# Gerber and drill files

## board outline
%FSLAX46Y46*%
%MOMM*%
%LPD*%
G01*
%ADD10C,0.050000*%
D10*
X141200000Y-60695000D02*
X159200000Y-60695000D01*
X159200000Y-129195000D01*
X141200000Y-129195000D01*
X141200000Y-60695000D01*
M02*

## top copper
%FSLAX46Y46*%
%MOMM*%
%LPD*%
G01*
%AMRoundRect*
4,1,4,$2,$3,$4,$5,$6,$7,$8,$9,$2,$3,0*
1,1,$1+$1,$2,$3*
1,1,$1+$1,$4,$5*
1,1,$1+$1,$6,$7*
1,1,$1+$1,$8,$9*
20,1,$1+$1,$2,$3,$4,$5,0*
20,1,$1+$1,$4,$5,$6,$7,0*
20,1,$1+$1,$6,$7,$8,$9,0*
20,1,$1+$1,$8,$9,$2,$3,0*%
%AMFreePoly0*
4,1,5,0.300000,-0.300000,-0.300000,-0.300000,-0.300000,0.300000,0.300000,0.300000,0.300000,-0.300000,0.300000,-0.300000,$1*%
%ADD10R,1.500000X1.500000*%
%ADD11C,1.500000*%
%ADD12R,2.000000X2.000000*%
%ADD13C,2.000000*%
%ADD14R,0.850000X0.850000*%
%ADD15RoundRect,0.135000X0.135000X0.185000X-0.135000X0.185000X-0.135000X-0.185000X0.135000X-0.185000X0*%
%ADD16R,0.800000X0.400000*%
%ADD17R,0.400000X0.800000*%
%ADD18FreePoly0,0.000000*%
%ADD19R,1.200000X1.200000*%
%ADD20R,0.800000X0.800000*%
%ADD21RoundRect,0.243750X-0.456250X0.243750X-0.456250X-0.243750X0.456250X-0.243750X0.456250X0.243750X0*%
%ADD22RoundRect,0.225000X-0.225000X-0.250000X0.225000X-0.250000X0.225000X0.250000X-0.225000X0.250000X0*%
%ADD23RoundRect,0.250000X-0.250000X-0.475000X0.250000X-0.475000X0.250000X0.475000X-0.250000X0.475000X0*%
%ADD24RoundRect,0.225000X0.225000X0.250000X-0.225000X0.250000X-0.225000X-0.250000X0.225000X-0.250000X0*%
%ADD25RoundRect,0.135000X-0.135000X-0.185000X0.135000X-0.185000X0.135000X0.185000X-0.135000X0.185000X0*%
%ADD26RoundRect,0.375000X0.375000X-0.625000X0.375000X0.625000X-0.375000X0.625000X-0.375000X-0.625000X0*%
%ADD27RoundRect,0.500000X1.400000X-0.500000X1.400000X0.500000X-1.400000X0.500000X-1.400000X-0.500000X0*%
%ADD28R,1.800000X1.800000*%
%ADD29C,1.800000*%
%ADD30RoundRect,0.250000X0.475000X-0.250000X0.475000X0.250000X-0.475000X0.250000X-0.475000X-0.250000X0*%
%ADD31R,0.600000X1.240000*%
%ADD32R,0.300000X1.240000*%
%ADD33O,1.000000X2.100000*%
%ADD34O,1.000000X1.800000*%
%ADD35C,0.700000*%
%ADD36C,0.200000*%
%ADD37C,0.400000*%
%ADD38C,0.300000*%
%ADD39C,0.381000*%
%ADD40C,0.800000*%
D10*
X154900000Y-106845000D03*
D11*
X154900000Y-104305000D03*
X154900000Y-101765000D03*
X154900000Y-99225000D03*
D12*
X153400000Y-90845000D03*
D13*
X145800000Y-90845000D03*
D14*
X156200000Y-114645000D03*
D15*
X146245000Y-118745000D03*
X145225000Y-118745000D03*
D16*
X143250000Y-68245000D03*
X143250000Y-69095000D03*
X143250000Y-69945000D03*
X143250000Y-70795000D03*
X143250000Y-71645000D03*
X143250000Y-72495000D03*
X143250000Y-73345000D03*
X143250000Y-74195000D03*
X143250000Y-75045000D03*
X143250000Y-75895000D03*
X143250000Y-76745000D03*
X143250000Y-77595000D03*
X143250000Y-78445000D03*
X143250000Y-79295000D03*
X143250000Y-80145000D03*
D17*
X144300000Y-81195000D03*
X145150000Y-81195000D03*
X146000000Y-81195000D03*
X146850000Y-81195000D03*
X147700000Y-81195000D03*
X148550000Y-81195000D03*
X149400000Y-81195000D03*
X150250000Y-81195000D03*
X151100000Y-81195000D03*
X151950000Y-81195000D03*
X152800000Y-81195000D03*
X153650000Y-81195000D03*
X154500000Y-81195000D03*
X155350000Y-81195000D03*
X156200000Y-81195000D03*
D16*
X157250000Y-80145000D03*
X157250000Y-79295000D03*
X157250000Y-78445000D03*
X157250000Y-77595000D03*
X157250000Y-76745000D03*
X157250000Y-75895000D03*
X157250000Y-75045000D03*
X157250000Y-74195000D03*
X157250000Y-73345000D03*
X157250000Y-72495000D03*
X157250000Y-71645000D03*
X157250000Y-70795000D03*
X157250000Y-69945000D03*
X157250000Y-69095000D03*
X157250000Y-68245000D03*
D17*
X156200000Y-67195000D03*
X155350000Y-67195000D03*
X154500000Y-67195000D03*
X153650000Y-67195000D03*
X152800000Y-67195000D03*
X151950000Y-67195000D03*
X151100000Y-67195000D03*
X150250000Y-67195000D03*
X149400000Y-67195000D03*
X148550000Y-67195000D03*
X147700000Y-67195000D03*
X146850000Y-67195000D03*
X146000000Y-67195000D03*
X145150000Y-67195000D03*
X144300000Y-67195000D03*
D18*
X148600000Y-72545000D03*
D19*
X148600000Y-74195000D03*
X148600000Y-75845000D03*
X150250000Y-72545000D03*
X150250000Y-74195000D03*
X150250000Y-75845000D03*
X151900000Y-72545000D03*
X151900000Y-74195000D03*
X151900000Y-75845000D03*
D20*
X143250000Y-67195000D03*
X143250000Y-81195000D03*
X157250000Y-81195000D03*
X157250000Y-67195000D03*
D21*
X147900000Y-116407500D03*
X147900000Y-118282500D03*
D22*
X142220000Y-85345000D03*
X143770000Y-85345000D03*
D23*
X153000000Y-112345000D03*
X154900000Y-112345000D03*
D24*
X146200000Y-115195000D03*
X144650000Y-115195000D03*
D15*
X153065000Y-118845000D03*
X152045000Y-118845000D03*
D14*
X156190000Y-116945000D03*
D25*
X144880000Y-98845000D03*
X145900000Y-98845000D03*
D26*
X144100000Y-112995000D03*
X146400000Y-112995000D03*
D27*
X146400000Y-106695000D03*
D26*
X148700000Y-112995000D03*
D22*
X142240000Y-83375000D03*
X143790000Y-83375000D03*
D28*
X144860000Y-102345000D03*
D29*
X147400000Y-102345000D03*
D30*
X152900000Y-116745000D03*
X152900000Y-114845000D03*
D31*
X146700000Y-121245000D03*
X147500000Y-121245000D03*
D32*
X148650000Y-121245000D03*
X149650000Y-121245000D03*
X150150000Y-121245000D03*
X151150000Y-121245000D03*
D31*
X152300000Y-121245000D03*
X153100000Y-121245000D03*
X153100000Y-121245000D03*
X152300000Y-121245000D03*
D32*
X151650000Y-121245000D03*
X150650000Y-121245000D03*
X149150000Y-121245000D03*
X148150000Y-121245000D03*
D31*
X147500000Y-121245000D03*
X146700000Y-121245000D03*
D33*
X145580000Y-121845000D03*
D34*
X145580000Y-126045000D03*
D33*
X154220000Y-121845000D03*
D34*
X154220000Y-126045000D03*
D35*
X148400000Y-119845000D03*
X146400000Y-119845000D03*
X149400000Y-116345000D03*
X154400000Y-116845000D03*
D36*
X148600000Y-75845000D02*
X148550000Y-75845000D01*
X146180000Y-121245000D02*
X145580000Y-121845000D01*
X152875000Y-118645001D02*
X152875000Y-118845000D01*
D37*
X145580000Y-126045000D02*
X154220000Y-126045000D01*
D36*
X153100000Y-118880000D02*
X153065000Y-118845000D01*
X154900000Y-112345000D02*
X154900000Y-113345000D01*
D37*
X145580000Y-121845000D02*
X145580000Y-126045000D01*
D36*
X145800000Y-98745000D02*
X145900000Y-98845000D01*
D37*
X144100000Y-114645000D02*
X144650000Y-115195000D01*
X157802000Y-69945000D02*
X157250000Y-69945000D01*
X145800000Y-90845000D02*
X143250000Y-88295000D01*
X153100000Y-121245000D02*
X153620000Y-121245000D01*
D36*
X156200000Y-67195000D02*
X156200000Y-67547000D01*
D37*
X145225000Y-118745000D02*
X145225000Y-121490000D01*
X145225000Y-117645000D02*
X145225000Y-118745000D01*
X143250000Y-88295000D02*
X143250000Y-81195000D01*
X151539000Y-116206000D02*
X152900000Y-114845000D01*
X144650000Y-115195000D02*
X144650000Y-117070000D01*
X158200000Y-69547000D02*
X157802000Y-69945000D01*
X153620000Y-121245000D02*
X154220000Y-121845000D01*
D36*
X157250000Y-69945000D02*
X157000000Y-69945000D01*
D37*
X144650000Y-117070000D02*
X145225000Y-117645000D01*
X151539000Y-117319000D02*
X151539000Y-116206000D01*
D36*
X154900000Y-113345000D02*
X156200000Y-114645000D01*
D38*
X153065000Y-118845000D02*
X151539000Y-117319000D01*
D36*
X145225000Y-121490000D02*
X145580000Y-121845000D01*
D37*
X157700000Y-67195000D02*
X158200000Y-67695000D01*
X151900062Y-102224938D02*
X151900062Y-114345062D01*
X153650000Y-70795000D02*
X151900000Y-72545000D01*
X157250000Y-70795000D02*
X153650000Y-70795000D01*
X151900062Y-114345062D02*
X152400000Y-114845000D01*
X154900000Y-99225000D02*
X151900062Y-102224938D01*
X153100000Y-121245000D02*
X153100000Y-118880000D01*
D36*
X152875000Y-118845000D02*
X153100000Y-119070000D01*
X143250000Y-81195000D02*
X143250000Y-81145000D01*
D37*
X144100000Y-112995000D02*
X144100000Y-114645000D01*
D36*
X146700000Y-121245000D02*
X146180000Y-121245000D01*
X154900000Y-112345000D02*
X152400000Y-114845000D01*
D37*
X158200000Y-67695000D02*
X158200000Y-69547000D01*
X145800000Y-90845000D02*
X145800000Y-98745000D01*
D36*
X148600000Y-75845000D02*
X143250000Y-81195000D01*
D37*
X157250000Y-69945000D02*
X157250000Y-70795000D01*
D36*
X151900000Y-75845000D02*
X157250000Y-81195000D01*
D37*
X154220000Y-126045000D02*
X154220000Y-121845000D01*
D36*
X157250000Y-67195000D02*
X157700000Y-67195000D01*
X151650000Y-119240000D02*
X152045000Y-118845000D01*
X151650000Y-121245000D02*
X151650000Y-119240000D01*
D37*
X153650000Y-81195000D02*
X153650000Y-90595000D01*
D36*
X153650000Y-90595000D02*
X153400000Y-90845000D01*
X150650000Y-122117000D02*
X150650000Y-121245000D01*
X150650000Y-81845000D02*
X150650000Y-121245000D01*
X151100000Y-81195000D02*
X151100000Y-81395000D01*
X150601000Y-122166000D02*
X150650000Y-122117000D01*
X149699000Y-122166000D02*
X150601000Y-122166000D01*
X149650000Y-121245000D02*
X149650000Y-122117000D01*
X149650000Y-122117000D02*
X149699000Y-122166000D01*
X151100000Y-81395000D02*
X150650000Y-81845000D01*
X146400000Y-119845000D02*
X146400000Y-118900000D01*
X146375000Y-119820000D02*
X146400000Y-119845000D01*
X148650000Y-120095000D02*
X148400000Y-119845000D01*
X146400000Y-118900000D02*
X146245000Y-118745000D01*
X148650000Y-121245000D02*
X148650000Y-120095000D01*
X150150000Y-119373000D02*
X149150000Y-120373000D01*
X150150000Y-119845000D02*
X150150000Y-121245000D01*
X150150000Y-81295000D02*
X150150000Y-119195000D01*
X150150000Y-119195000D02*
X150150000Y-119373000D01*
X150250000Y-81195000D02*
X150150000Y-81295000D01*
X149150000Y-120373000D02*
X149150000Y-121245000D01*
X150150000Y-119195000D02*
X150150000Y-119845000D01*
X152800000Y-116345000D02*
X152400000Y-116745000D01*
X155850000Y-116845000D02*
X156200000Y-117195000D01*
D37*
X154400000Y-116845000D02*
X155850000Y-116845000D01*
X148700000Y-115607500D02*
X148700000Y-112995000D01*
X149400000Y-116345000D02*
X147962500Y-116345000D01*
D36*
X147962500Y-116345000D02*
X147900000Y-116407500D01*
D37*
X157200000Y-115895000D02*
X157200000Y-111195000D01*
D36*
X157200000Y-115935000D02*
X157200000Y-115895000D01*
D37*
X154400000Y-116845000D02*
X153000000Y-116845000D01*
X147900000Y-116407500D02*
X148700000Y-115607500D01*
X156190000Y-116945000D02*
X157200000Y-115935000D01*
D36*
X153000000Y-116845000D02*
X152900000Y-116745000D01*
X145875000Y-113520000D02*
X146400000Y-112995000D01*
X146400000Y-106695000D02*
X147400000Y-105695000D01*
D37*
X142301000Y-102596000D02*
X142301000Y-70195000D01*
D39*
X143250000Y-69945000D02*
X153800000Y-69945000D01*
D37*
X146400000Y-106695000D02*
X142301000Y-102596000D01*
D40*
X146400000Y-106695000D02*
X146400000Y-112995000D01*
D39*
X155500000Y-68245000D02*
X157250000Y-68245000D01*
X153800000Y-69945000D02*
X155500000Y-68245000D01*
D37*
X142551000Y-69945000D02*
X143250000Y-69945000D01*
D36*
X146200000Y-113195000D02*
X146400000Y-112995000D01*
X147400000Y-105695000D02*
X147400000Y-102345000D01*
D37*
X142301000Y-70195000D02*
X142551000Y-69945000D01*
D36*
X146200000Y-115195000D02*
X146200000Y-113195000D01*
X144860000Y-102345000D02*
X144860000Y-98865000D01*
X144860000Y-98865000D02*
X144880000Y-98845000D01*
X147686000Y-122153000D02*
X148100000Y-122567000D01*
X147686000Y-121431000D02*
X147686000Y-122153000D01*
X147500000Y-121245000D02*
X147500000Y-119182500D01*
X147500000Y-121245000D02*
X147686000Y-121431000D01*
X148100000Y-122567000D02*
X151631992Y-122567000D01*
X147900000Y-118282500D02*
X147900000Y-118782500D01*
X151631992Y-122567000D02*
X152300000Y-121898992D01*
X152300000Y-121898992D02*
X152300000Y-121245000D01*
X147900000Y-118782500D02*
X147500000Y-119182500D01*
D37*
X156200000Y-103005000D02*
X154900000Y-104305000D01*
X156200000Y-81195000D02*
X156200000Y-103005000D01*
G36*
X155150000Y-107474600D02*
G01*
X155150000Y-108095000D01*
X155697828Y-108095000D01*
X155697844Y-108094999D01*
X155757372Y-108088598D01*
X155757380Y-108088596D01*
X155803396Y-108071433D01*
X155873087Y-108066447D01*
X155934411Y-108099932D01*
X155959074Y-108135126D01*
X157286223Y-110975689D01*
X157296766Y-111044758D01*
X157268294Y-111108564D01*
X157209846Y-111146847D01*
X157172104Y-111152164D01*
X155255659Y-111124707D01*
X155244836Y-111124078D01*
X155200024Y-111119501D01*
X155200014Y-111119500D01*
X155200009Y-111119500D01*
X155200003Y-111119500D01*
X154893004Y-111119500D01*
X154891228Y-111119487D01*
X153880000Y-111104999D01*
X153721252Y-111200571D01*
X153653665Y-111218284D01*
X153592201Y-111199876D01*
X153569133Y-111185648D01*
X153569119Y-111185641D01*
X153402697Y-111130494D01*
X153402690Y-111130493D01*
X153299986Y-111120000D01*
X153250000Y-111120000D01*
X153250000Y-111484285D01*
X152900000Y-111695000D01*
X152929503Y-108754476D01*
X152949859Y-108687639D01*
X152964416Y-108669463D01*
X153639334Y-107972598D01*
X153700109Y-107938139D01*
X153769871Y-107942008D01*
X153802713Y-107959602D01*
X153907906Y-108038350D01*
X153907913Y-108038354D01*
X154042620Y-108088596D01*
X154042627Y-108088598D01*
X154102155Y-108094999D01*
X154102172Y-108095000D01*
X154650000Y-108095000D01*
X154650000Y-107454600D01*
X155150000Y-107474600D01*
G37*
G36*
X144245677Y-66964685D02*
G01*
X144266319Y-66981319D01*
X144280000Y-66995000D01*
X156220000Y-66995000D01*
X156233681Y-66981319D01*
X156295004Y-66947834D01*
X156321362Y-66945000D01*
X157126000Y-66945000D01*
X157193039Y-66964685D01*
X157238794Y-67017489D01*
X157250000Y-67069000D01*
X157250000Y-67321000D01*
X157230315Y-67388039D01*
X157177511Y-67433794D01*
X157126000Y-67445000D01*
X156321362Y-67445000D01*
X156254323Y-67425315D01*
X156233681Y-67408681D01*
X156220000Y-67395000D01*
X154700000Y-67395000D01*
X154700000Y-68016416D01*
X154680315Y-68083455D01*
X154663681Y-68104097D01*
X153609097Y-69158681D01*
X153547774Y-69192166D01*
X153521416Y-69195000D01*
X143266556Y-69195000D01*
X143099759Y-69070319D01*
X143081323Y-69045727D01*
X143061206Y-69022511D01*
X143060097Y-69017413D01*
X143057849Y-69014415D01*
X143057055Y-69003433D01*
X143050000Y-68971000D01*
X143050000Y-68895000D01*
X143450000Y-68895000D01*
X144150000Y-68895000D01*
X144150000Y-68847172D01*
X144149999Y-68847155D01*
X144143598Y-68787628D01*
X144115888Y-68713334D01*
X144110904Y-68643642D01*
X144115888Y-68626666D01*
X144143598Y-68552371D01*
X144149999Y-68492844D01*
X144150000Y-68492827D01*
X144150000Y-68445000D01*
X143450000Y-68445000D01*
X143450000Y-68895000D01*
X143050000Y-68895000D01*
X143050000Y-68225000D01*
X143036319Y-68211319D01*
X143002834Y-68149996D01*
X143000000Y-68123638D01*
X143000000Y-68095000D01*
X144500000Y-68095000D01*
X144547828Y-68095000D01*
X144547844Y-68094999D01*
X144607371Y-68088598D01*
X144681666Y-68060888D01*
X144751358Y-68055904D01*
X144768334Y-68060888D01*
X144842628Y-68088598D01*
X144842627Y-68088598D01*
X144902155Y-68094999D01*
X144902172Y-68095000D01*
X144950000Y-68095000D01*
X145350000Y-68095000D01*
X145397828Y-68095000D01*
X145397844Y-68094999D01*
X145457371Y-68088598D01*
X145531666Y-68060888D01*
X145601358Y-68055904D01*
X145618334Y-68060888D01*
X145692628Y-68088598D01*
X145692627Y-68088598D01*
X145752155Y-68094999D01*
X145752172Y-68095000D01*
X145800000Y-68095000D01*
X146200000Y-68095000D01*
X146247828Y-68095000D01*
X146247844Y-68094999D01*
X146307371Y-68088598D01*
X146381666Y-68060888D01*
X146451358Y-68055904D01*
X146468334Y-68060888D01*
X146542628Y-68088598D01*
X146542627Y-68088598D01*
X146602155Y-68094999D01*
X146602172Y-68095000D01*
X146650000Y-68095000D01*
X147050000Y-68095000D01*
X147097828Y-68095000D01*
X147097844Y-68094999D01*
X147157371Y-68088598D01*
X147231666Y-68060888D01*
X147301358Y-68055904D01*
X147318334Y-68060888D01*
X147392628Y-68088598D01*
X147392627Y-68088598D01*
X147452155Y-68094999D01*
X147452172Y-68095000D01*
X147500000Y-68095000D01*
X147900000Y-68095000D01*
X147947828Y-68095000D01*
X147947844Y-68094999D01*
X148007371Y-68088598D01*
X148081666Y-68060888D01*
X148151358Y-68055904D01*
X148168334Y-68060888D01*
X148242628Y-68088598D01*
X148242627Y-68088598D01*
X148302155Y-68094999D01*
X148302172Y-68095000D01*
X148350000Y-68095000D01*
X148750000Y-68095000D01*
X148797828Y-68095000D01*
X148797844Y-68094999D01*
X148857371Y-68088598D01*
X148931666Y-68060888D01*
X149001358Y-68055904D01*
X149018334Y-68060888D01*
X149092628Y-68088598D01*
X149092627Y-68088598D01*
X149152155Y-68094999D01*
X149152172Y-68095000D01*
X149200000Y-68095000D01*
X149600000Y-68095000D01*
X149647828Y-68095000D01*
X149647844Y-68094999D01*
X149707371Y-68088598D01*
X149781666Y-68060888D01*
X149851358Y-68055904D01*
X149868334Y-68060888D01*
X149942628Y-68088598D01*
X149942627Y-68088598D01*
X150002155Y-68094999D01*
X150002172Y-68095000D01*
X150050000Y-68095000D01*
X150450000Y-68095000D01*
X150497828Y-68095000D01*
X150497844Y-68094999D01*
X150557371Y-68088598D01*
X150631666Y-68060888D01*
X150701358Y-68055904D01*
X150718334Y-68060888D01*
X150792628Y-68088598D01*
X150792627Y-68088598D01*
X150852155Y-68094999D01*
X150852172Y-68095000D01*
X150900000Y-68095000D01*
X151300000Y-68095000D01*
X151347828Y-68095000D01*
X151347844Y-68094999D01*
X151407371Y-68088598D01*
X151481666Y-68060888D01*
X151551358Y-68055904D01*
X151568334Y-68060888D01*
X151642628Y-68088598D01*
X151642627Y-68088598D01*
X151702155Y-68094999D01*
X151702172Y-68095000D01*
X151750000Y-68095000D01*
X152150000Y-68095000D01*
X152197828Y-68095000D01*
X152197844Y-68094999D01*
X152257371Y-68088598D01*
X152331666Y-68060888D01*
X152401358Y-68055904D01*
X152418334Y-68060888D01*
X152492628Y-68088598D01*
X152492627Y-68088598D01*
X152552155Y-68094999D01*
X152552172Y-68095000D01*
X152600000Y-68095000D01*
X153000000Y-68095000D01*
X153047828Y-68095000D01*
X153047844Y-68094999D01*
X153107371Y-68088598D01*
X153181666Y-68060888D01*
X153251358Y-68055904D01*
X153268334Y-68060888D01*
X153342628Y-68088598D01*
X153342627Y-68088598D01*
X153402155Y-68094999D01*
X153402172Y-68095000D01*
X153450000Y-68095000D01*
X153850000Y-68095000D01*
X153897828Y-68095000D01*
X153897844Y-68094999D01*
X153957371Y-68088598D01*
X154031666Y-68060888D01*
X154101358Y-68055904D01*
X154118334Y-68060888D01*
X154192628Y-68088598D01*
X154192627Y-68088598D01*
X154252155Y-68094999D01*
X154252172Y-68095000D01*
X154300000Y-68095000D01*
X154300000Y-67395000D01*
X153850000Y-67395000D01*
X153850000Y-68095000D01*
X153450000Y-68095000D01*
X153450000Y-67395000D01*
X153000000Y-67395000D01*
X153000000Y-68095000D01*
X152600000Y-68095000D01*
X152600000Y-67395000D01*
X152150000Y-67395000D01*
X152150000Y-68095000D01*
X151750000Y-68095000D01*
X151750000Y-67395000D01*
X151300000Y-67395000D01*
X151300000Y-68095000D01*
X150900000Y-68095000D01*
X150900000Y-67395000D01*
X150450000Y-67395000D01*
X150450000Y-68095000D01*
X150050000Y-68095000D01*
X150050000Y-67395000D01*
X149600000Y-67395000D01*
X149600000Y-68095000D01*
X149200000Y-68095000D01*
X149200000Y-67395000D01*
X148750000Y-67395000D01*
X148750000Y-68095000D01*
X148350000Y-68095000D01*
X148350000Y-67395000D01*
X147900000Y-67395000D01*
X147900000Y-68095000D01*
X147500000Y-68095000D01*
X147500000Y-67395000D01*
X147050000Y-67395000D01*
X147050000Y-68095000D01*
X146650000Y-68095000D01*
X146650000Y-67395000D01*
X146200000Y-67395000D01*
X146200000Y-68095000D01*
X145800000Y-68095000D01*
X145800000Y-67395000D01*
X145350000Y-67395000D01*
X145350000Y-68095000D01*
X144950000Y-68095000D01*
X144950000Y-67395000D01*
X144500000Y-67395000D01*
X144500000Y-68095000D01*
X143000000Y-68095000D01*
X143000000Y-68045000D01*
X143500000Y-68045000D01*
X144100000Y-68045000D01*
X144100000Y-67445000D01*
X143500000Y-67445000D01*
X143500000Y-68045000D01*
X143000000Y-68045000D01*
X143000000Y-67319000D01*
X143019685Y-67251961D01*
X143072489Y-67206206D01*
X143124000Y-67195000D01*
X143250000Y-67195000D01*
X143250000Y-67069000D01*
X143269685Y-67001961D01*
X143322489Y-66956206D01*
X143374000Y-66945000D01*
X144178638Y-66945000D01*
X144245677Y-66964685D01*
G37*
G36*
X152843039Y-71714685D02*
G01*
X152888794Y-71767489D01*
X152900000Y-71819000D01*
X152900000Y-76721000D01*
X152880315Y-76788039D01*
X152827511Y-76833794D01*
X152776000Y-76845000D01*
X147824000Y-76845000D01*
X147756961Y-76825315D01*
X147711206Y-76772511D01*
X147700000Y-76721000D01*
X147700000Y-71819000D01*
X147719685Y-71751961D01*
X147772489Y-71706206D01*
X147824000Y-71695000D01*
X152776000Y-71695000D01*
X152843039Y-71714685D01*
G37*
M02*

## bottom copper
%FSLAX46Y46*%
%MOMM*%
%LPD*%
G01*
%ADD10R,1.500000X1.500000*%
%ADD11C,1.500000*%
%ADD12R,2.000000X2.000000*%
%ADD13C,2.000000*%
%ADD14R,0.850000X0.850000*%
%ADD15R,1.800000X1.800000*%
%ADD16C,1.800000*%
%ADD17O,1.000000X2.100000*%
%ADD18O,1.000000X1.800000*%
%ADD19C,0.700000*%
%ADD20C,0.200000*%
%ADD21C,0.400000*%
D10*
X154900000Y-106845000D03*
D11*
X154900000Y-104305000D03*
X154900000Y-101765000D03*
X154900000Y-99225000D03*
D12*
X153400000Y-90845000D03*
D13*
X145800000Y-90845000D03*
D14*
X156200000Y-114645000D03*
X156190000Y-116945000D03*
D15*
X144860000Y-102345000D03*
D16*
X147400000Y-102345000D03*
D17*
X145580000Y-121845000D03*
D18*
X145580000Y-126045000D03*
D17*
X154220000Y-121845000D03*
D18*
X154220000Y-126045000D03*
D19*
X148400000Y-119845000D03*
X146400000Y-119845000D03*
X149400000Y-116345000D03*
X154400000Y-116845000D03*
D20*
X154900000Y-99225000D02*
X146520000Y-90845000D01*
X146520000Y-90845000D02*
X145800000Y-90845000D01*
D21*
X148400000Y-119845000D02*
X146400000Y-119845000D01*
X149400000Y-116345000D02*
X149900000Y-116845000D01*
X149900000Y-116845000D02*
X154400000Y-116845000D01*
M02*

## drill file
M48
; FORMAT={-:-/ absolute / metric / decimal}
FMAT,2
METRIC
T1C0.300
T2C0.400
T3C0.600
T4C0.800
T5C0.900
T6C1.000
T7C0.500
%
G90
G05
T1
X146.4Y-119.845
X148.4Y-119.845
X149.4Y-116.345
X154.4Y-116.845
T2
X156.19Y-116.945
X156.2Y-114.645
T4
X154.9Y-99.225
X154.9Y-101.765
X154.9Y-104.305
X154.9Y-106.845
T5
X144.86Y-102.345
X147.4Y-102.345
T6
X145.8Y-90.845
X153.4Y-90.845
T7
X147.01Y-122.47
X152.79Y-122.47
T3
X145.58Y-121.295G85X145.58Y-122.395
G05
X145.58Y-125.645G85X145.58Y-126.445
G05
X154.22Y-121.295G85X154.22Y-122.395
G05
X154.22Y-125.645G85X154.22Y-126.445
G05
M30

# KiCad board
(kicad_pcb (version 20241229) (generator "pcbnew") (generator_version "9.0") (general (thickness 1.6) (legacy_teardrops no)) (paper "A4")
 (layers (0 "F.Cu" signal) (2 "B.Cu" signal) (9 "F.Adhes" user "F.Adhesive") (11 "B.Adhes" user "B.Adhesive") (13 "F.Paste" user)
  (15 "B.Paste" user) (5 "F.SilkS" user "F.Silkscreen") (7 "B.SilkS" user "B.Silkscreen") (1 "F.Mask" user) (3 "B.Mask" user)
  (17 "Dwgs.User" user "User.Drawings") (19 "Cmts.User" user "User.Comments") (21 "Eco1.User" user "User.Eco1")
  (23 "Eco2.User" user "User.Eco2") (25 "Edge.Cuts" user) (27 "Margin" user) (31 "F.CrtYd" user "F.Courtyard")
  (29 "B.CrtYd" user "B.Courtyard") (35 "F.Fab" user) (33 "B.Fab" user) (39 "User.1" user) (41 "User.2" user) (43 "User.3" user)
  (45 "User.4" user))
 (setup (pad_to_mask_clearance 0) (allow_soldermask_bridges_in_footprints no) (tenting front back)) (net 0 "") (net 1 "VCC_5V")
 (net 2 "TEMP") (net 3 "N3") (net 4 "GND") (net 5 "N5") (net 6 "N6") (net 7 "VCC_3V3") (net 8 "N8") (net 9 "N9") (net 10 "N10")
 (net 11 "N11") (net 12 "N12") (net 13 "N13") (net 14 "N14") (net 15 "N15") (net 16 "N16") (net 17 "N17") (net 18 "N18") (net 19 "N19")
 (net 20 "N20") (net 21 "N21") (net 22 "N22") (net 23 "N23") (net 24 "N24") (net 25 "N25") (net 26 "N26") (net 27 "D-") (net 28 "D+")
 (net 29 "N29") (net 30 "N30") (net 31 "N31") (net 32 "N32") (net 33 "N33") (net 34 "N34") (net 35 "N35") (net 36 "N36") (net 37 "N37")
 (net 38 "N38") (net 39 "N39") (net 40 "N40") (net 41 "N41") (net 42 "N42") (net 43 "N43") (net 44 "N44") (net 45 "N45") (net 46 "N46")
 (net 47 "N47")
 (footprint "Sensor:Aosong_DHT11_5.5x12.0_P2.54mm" (layer "F.Cu") (at 154.9 106.845 180)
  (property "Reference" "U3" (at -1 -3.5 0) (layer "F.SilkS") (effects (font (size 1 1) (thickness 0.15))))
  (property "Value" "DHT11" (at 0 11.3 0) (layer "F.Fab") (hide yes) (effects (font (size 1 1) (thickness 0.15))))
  (pad "1" thru_hole rect (at 0 0 180) (size 1.5 1.5) (drill 0.8) (layers "*.Cu" "*.Mask") (remove_unused_layers no) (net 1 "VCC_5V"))
  (pad "2" thru_hole circle (at 0 2.54 180) (size 1.5 1.5) (drill 0.8) (layers "*.Cu" "*.Mask") (remove_unused_layers no) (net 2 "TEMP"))
  (pad "3" thru_hole circle (at 0 5.08 180) (size 1.5 1.5) (drill 0.8) (layers "*.Cu" "*.Mask") (remove_unused_layers no) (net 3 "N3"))
  (pad "4" thru_hole circle (at 0 7.62 180) (size 1.5 1.5) (drill 0.8) (layers "*.Cu" "*.Mask") (remove_unused_layers no) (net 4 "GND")))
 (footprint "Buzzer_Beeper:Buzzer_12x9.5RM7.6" (layer "F.Cu") (at 153.4 90.845 180)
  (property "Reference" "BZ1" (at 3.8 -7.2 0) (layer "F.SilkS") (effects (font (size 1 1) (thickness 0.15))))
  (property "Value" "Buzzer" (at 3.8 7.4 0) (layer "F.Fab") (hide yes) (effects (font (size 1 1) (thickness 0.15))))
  (pad "1" thru_hole rect (at 0 0 180) (size 2 2) (drill 1) (layers "*.Cu" "*.Mask") (remove_unused_layers no) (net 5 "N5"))
  (pad "2" thru_hole circle (at 7.6 0 180) (size 2 2) (drill 1) (layers "*.Cu" "*.Mask") (remove_unused_layers no) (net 4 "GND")))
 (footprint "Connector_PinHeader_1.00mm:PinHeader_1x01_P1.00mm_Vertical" (layer "F.Cu") (at 156.2 114.645)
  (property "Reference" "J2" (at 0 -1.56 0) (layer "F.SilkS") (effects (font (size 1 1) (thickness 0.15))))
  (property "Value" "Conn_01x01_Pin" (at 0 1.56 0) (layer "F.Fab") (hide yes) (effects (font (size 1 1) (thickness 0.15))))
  (pad "1" thru_hole rect (at 0 0) (size 0.85 0.85) (drill 0.4) (layers "*.Cu" "*.Mask") (remove_unused_layers no) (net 4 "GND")))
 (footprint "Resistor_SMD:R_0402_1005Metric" (layer "F.Cu") (at 145.735 118.745 180)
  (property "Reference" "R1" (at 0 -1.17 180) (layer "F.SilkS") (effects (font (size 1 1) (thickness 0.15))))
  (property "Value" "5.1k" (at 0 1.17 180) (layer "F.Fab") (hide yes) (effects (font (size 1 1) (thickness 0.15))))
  (pad "1" smd roundrect (at -0.51 0 180) (size 0.54 0.64) (layers "F.Cu" "F.Mask" "F.Paste") (roundrect_rratio 0.25) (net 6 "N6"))
  (pad "2" smd roundrect (at 0.51 0 180) (size 0.54 0.64) (layers "F.Cu" "F.Mask" "F.Paste") (roundrect_rratio 0.25) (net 4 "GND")))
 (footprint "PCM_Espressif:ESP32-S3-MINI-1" (layer "F.Cu") (at 150.25 74.195)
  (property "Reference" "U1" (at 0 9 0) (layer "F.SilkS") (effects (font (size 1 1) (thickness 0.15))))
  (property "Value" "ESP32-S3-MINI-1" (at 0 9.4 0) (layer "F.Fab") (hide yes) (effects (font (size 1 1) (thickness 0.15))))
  (pad "1" smd rect (at -7 -5.95 90) (size 0.4 0.8) (layers "F.Cu" "F.Mask" "F.Paste") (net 4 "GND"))
  (pad "2" smd rect (at -7 -5.1 90) (size 0.4 0.8) (layers "F.Cu" "F.Mask" "F.Paste") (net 4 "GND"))
  (pad "3" smd rect (at -7 -4.25 90) (size 0.4 0.8) (layers "F.Cu" "F.Mask" "F.Paste") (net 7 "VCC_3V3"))
  (pad "4" smd rect (at -7 -3.4 90) (size 0.4 0.8) (layers "F.Cu" "F.Mask" "F.Paste") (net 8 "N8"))
  (pad "5" smd rect (at -7 -2.55 90) (size 0.4 0.8) (layers "F.Cu" "F.Mask" "F.Paste") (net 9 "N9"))
  (pad "6" smd rect (at -7 -1.7 90) (size 0.4 0.8) (layers "F.Cu" "F.Mask" "F.Paste") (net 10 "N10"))
  (pad "7" smd rect (at -7 -0.85 90) (size 0.4 0.8) (layers "F.Cu" "F.Mask" "F.Paste") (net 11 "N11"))
  (pad "8" smd rect (at -7 0 90) (size 0.4 0.8) (layers "F.Cu" "F.Mask" "F.Paste") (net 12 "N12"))
  (pad "9" smd rect (at -7 0.85 90) (size 0.4 0.8) (layers "F.Cu" "F.Mask" "F.Paste") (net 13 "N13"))
  (pad "10" smd rect (at -7 1.7 90) (size 0.4 0.8) (layers "F.Cu" "F.Mask" "F.Paste") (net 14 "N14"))
  (pad "11" smd rect (at -7 2.55 90) (size 0.4 0.8) (layers "F.Cu" "F.Mask" "F.Paste") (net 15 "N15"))
  (pad "12" smd rect (at -7 3.4 90) (size 0.4 0.8) (layers "F.Cu" "F.Mask" "F.Paste") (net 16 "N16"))
  (pad "13" smd rect (at -7 4.25 90) (size 0.4 0.8) (layers "F.Cu" "F.Mask" "F.Paste") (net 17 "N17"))
  (pad "14" smd rect (at -7 5.1 90) (size 0.4 0.8) (layers "F.Cu" "F.Mask" "F.Paste") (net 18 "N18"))
  (pad "15" smd rect (at -7 5.95 90) (size 0.4 0.8) (layers "F.Cu" "F.Mask" "F.Paste") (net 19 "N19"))
  (pad "16" smd rect (at -5.95 7) (size 0.4 0.8) (layers "F.Cu" "F.Mask" "F.Paste") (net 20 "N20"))
  (pad "17" smd rect (at -5.1 7) (size 0.4 0.8) (layers "F.Cu" "F.Mask" "F.Paste") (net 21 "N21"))
  (pad "18" smd rect (at -4.25 7) (size 0.4 0.8) (layers "F.Cu" "F.Mask" "F.Paste") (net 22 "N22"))
  (pad "19" smd rect (at -3.4 7) (size 0.4 0.8) (layers "F.Cu" "F.Mask" "F.Paste") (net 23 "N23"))
  (pad "20" smd rect (at -2.55 7) (size 0.4 0.8) (layers "F.Cu" "F.Mask" "F.Paste") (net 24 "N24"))
  (pad "21" smd rect (at -1.7 7) (size 0.4 0.8) (layers "F.Cu" "F.Mask" "F.Paste") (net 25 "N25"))
  (pad "22" smd rect (at -0.85 7) (size 0.4 0.8) (layers "F.Cu" "F.Mask" "F.Paste") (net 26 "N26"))
  (pad "23" smd rect (at 0 7) (size 0.4 0.8) (layers "F.Cu" "F.Mask" "F.Paste") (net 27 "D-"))
  (pad "24" smd rect (at 0.85 7) (size 0.4 0.8) (layers "F.Cu" "F.Mask" "F.Paste") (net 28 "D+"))
  (pad "25" smd rect (at 1.7 7) (size 0.4 0.8) (layers "F.Cu" "F.Mask" "F.Paste") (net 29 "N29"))
  (pad "26" smd rect (at 2.55 7) (size 0.4 0.8) (layers "F.Cu" "F.Mask" "F.Paste") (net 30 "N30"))
  (pad "27" smd rect (at 3.4 7) (size 0.4 0.8) (layers "F.Cu" "F.Mask" "F.Paste") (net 5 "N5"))
  (pad "28" smd rect (at 4.25 7) (size 0.4 0.8) (layers "F.Cu" "F.Mask" "F.Paste") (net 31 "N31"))
  (pad "29" smd rect (at 5.1 7) (size 0.4 0.8) (layers "F.Cu" "F.Mask" "F.Paste") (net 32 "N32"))
  (pad "30" smd rect (at 5.95 7) (size 0.4 0.8) (layers "F.Cu" "F.Mask" "F.Paste") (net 2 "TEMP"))
  (pad "31" smd rect (at 7 5.95 90) (size 0.4 0.8) (layers "F.Cu" "F.Mask" "F.Paste") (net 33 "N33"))
  (pad "32" smd rect (at 7 5.1 90) (size 0.4 0.8) (layers "F.Cu" "F.Mask" "F.Paste") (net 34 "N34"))
  (pad "33" smd rect (at 7 4.25 90) (size 0.4 0.8) (layers "F.Cu" "F.Mask" "F.Paste") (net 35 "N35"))
  (pad "34" smd rect (at 7 3.4 90) (size 0.4 0.8) (layers "F.Cu" "F.Mask" "F.Paste") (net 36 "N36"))
  (pad "35" smd rect (at 7 2.55 90) (size 0.4 0.8) (layers "F.Cu" "F.Mask" "F.Paste") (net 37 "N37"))
  (pad "36" smd rect (at 7 1.7 90) (size 0.4 0.8) (layers "F.Cu" "F.Mask" "F.Paste") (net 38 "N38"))
  (pad "37" smd rect (at 7 0.85 90) (size 0.4 0.8) (layers "F.Cu" "F.Mask" "F.Paste") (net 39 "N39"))
  (pad "38" smd rect (at 7 0 90) (size 0.4 0.8) (layers "F.Cu" "F.Mask" "F.Paste") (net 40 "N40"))
  (pad "39" smd rect (at 7 -0.85 90) (size 0.4 0.8) (layers "F.Cu" "F.Mask" "F.Paste") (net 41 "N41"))
  (pad "40" smd rect (at 7 -1.7 90) (size 0.4 0.8) (layers "F.Cu" "F.Mask" "F.Paste") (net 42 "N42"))
  (pad "41" smd rect (at 7 -2.55 90) (size 0.4 0.8) (layers "F.Cu" "F.Mask" "F.Paste") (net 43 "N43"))
  (pad "42" smd rect (at 7 -3.4 90) (size 0.4 0.8) (layers "F.Cu" "F.Mask" "F.Paste") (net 4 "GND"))
  (pad "43" smd rect (at 7 -4.25 90) (size 0.4 0.8) (layers "F.Cu" "F.Mask" "F.Paste") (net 4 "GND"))
  (pad "44" smd rect (at 7 -5.1 90) (size 0.4 0.8) (layers "F.Cu" "F.Mask" "F.Paste") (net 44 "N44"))
  (pad "45" smd rect (at 7 -5.95 90) (size 0.4 0.8) (layers "F.Cu" "F.Mask" "F.Paste") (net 7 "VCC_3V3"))
  (pad "46" smd rect (at 5.95 -7) (size 0.4 0.8) (layers "F.Cu" "F.Mask" "F.Paste") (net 4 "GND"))
  (pad "47" smd rect (at 5.1 -7) (size 0.4 0.8) (layers "F.Cu" "F.Mask" "F.Paste") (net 4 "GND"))
  (pad "48" smd rect (at 4.25 -7) (size 0.4 0.8) (layers "F.Cu" "F.Mask" "F.Paste") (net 4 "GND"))
  (pad "49" smd rect (at 3.4 -7) (size 0.4 0.8) (layers "F.Cu" "F.Mask" "F.Paste") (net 4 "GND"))
  (pad "50" smd rect (at 2.55 -7) (size 0.4 0.8) (layers "F.Cu" "F.Mask" "F.Paste") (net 4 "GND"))
  (pad "51" smd rect (at 1.7 -7) (size 0.4 0.8) (layers "F.Cu" "F.Mask" "F.Paste") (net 4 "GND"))
  (pad "52" smd rect (at 0.85 -7) (size 0.4 0.8) (layers "F.Cu" "F.Mask" "F.Paste") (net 4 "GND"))
  (pad "53" smd rect (at 0 -7) (size 0.4 0.8) (layers "F.Cu" "F.Mask" "F.Paste") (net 4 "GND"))
  (pad "54" smd rect (at -0.85 -7) (size 0.4 0.8) (layers "F.Cu" "F.Mask" "F.Paste") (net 4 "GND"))
  (pad "55" smd rect (at -1.7 -7) (size 0.4 0.8) (layers "F.Cu" "F.Mask" "F.Paste") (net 4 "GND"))
  (pad "56" smd rect (at -2.55 -7) (size 0.4 0.8) (layers "F.Cu" "F.Mask" "F.Paste") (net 4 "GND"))
  (pad "57" smd rect (at -3.4 -7) (size 0.4 0.8) (layers "F.Cu" "F.Mask" "F.Paste") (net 4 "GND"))
  (pad "58" smd rect (at -4.25 -7) (size 0.4 0.8) (layers "F.Cu" "F.Mask" "F.Paste") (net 4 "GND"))
  (pad "59" smd rect (at -5.1 -7) (size 0.4 0.8) (layers "F.Cu" "F.Mask" "F.Paste") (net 4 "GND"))
  (pad "60" smd rect (at -5.95 -7) (size 0.4 0.8) (layers "F.Cu" "F.Mask" "F.Paste") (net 4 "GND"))
  (pad "61" smd custom (at -1.65 -1.65) (size 0.6 0.6) (layers "F.Cu" "F.Mask" "F.Paste") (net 4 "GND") (zone_connect 2)
   (thermal_bridge_angle 45) (options (clearance outline) (anchor rect)) (primitives))
  (pad "61" smd rect (at -1.65 0) (size 1.2 1.2) (layers "F.Cu" "F.Mask" "F.Paste") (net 4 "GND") (zone_connect 2))
  (pad "61" smd rect (at -1.65 1.65) (size 1.2 1.2) (layers "F.Cu" "F.Mask" "F.Paste") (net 4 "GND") (zone_connect 2))
  (pad "61" smd rect (at 0 -1.65) (size 1.2 1.2) (layers "F.Cu" "F.Mask" "F.Paste") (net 4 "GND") (zone_connect 2))
  (pad "61" smd rect (at 0 0) (size 1.2 1.2) (layers "F.Cu" "F.Mask" "F.Paste") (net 4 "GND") (zone_connect 2))
  (pad "61" smd rect (at 0 1.65) (size 1.2 1.2) (layers "F.Cu" "F.Mask" "F.Paste") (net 4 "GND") (zone_connect 2))
  (pad "61" smd rect (at 1.65 -1.65) (size 1.2 1.2) (layers "F.Cu" "F.Mask" "F.Paste") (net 4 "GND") (zone_connect 2))
  (pad "61" smd rect (at 1.65 0) (size 1.2 1.2) (layers "F.Cu" "F.Mask" "F.Paste") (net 4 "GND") (zone_connect 2))
  (pad "61" smd rect (at 1.65 1.65) (size 1.2 1.2) (layers "F.Cu" "F.Mask" "F.Paste") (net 4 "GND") (zone_connect 2))
  (pad "62" smd rect (at -7 -7 180) (size 0.8 0.8) (layers "F.Cu" "F.Mask" "F.Paste") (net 4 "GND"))
  (pad "63" smd rect (at -7 7 180) (size 0.8 0.8) (layers "F.Cu" "F.Mask" "F.Paste") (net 4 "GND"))
  (pad "64" smd rect (at 7 7 180) (size 0.8 0.8) (layers "F.Cu" "F.Mask" "F.Paste") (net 4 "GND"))
  (pad "65" smd rect (at 7 -7 180) (size 0.8 0.8) (layers "F.Cu" "F.Mask" "F.Paste") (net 4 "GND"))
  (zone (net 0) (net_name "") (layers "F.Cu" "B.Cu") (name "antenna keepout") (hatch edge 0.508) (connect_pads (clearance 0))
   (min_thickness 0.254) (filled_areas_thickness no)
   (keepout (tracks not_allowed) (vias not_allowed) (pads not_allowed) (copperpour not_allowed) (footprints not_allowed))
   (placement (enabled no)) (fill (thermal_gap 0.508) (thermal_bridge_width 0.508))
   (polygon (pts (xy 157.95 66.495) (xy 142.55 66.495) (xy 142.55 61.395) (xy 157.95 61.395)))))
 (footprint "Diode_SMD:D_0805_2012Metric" (layer "F.Cu") (at 147.9 117.345 -90)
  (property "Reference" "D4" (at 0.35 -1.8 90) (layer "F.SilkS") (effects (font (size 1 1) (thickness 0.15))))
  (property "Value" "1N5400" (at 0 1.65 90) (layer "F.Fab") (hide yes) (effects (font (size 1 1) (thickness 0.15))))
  (pad "1" smd roundrect (at -0.9375 0 270) (size 0.975 1.4) (layers "F.Cu" "F.Mask" "F.Paste") (roundrect_rratio 0.25) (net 1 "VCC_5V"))
  (pad "2" smd roundrect (at 0.9375 0 270) (size 0.975 1.4) (layers "F.Cu" "F.Mask" "F.Paste") (roundrect_rratio 0.25) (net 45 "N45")))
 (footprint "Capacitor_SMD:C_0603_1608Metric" (layer "F.Cu") (at 142.995 85.345)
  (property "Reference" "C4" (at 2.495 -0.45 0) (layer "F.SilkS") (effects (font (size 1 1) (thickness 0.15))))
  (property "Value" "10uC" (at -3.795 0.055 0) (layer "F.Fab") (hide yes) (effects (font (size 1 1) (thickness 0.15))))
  (pad "1" smd roundrect (at -0.775 0) (size 0.9 0.95) (layers "F.Cu" "F.Mask" "F.Paste") (roundrect_rratio 0.25) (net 7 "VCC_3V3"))
  (pad "2" smd roundrect (at 0.775 0) (size 0.9 0.95) (layers "F.Cu" "F.Mask" "F.Paste") (roundrect_rratio 0.25) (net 4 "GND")))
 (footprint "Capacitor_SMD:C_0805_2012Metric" (layer "F.Cu") (at 153.95 112.345)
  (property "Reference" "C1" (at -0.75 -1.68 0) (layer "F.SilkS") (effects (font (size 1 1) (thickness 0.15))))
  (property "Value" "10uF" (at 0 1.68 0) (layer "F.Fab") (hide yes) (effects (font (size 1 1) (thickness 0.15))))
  (pad "1" smd roundrect (at -0.95 0) (size 1 1.45) (layers "F.Cu" "F.Mask" "F.Paste") (roundrect_rratio 0.25) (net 1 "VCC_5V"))
  (pad "2" smd roundrect (at 0.95 0) (size 1 1.45) (layers "F.Cu" "F.Mask" "F.Paste") (roundrect_rratio 0.25) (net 4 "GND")))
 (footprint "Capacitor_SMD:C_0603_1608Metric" (layer "F.Cu") (at 145.425 115.195 180)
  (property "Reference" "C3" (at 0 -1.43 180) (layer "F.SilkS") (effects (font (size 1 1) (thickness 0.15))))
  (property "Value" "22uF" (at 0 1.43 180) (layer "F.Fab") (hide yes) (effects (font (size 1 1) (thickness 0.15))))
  (pad "1" smd roundrect (at -0.775 0 180) (size 0.9 0.95) (layers "F.Cu" "F.Mask" "F.Paste") (roundrect_rratio 0.25) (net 7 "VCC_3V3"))
  (pad "2" smd roundrect (at 0.775 0 180) (size 0.9 0.95) (layers "F.Cu" "F.Mask" "F.Paste") (roundrect_rratio 0.25) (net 4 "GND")))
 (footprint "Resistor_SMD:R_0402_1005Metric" (layer "F.Cu") (at 152.555 118.845 180)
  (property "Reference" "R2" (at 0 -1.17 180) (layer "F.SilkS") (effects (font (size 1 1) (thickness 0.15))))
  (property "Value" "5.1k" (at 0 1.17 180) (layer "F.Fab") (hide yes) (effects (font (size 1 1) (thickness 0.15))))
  (pad "1" smd roundrect (at -0.51 0 180) (size 0.54 0.64) (layers "F.Cu" "F.Mask" "F.Paste") (roundrect_rratio 0.25) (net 4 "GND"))
  (pad "2" smd roundrect (at 0.51 0 180) (size 0.54 0.64) (layers "F.Cu" "F.Mask" "F.Paste") (roundrect_rratio 0.25) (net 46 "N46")))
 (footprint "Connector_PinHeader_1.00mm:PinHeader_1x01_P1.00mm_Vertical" (layer "F.Cu") (at 156.19 116.945)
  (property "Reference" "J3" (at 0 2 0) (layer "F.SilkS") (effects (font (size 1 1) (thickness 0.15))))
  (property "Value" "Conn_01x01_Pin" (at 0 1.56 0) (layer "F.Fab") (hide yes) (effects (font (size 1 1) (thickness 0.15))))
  (pad "1" thru_hole rect (at 0 0) (size 0.85 0.85) (drill 0.4) (layers "*.Cu" "*.Mask") (remove_unused_layers no) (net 1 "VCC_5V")))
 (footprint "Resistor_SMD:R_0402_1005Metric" (layer "F.Cu") (at 145.39 98.845)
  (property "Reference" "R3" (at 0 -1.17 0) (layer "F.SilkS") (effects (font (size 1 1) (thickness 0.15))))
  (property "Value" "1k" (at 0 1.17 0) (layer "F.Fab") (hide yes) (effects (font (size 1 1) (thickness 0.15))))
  (pad "1" smd roundrect (at -0.51 0) (size 0.54 0.64) (layers "F.Cu" "F.Mask" "F.Paste") (roundrect_rratio 0.25) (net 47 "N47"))
  (pad "2" smd roundrect (at 0.51 0) (size 0.54 0.64) (layers "F.Cu" "F.Mask" "F.Paste") (roundrect_rratio 0.25) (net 4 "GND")))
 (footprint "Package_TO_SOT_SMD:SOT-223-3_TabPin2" (layer "F.Cu") (at 146.4 109.845 90)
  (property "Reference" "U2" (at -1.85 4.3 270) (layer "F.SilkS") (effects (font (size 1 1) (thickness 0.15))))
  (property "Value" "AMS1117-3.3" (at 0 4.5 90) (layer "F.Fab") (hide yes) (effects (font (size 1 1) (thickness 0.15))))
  (pad "1" smd roundrect (at -3.15 -2.3 90) (size 2 1.5) (layers "F.Cu" "F.Mask" "F.Paste") (roundrect_rratio 0.25) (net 4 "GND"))
  (pad "2" smd roundrect (at -3.15 0 90) (size 2 1.5) (layers "F.Cu" "F.Mask" "F.Paste") (roundrect_rratio 0.25) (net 7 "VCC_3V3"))
  (pad "2" smd roundrect (at 3.15 0 90) (size 2 3.8) (layers "F.Cu" "F.Mask" "F.Paste") (roundrect_rratio 0.25) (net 7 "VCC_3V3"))
  (pad "3" smd roundrect (at -3.15 2.3 90) (size 2 1.5) (layers "F.Cu" "F.Mask" "F.Paste") (roundrect_rratio 0.25) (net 1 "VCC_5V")))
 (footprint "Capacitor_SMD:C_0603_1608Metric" (layer "F.Cu") (at 143.015 83.375)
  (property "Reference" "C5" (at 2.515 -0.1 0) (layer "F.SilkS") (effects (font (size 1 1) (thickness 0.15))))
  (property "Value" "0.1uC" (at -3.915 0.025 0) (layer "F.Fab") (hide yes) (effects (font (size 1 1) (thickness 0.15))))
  (pad "1" smd roundrect (at -0.775 0) (size 0.9 0.95) (layers "F.Cu" "F.Mask" "F.Paste") (roundrect_rratio 0.25) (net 7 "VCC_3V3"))
  (pad "2" smd roundrect (at 0.775 0) (size 0.9 0.95) (layers "F.Cu" "F.Mask" "F.Paste") (roundrect_rratio 0.25) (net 4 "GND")))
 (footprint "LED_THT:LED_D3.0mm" (layer "F.Cu") (at 144.86 102.345)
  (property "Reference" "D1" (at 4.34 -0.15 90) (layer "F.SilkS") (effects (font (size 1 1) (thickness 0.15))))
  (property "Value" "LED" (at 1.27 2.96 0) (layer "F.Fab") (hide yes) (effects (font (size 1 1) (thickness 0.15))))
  (pad "1" thru_hole rect (at 0 0) (size 1.8 1.8) (drill 0.9) (layers "*.Cu" "*.Mask") (remove_unused_layers no) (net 47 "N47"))
  (pad "2" thru_hole circle (at 2.54 0) (size 1.8 1.8) (drill 0.9) (layers "*.Cu" "*.Mask") (remove_unused_layers no) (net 7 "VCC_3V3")))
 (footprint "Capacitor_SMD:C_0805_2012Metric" (layer "F.Cu") (at 152.9 115.795 90)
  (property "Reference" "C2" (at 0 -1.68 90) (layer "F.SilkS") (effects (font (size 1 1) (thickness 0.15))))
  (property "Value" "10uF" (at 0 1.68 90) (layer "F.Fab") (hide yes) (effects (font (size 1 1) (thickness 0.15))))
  (pad "1" smd roundrect (at -0.95 0 90) (size 1 1.45) (layers "F.Cu" "F.Mask" "F.Paste") (roundrect_rratio 0.25) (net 1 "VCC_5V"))
  (pad "2" smd roundrect (at 0.95 0 90) (size 1 1.45) (layers "F.Cu" "F.Mask" "F.Paste") (roundrect_rratio 0.25) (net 4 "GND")))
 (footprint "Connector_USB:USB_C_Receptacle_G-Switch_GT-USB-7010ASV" (layer "F.Cu") (at 149.9 124.97)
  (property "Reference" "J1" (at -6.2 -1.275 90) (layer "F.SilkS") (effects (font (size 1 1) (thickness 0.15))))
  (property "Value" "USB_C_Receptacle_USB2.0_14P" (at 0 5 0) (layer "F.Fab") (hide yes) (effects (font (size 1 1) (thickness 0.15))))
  (pad "" np_thru_hole circle (at -2.89 -2.5) (size 0.5 0.5) (drill 0.5) (layers "*.Cu" "*.Mask"))
  (pad "" np_thru_hole circle (at 2.89 -2.5) (size 0.5 0.5) (drill 0.5) (layers "*.Cu" "*.Mask"))
  (pad "A1" smd rect (at -3.2 -3.725) (size 0.6 1.24) (layers "F.Cu" "F.Mask" "F.Paste") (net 4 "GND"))
  (pad "A4" smd rect (at -2.4 -3.725) (size 0.6 1.24) (layers "F.Cu" "F.Mask" "F.Paste") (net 45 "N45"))
  (pad "A5" smd rect (at -1.25 -3.725) (size 0.3 1.24) (layers "F.Cu" "F.Mask" "F.Paste") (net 6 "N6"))
  (pad "A6" smd rect (at -0.25 -3.725) (size 0.3 1.24) (layers "F.Cu" "F.Mask" "F.Paste") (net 28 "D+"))
  (pad "A7" smd rect (at 0.25 -3.725) (size 0.3 1.24) (layers "F.Cu" "F.Mask" "F.Paste") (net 27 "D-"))
  (pad "A8" smd rect (at 1.25 -3.725) (size 0.3 1.24) (layers "F.Cu" "F.Mask" "F.Paste"))
  (pad "A9" smd rect (at 2.4 -3.725) (size 0.6 1.24) (layers "F.Cu" "F.Mask" "F.Paste") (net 45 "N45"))
  (pad "A12" smd rect (at 3.2 -3.725) (size 0.6 1.24) (layers "F.Cu" "F.Mask" "F.Paste") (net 4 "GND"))
  (pad "B1" smd rect (at 3.2 -3.725) (size 0.6 1.24) (layers "F.Cu" "F.Mask" "F.Paste") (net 4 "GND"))
  (pad "B4" smd rect (at 2.4 -3.725) (size 0.6 1.24) (layers "F.Cu" "F.Mask" "F.Paste") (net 45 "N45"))
  (pad "B5" smd rect (at 1.75 -3.725) (size 0.3 1.24) (layers "F.Cu" "F.Mask" "F.Paste") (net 46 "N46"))
  (pad "B6" smd rect (at 0.75 -3.725) (size 0.3 1.24) (layers "F.Cu" "F.Mask" "F.Paste") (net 28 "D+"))
  (pad "B7" smd rect (at -0.75 -3.725) (size 0.3 1.24) (layers "F.Cu" "F.Mask" "F.Paste") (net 27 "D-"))
  (pad "B8" smd rect (at -1.75 -3.725) (size 0.3 1.24) (layers "F.Cu" "F.Mask" "F.Paste"))
  (pad "B9" smd rect (at -2.4 -3.725) (size 0.6 1.24) (layers "F.Cu" "F.Mask" "F.Paste") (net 45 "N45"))
  (pad "B12" smd rect (at -3.2 -3.725) (size 0.6 1.24) (layers "F.Cu" "F.Mask" "F.Paste") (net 4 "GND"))
  (pad "S1" thru_hole oval (at -4.32 -3.125) (size 1 2.1) (drill oval 0.6 1.7) (layers "*.Cu" "*.Mask") (remove_unused_layers no)
   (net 4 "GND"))
  (pad "S1" thru_hole oval (at -4.32 1.075) (size 1 1.8) (drill oval 0.6 1.4) (layers "*.Cu" "*.Mask") (remove_unused_layers no)
   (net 4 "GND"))
  (pad "S1" thru_hole oval (at 4.32 -3.125) (size 1 2.1) (drill oval 0.6 1.7) (layers "*.Cu" "*.Mask") (remove_unused_layers no)
   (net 4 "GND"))
  (pad "S1" thru_hole oval (at 4.32 1.075) (size 1 1.8) (drill oval 0.6 1.4) (layers "*.Cu" "*.Mask") (remove_unused_layers no)
   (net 4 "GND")))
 (gr_rect (start 141.2 60.695) (end 159.2 129.195) (stroke (width 0.05) (type default)) (fill no) (layer "Edge.Cuts"))
 (segment (start 148.6 75.845) (end 148.55 75.845) (width 0.2) (layer "F.Cu") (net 4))
 (segment (start 146.18 121.245) (end 145.58 121.845) (width 0.2) (layer "F.Cu") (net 4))
 (segment (start 152.875 118.645001) (end 152.875 118.845) (width 0.2) (layer "F.Cu") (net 4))
 (segment (start 145.58 126.045) (end 154.22 126.045) (width 0.4) (layer "F.Cu") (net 4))
 (segment (start 153.1 118.88) (end 153.065 118.845) (width 0.2) (layer "F.Cu") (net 4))
 (segment (start 154.9 112.345) (end 154.9 113.345) (width 0.2) (layer "F.Cu") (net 4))
 (segment (start 145.58 121.845) (end 145.58 126.045) (width 0.4) (layer "F.Cu") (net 4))
 (segment (start 145.8 98.745) (end 145.9 98.845) (width 0.2) (layer "F.Cu") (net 4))
 (segment (start 144.1 114.645) (end 144.65 115.195) (width 0.4) (layer "F.Cu") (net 4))
 (segment (start 157.802 69.945) (end 157.25 69.945) (width 0.4) (layer "F.Cu") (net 4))
 (segment (start 145.8 90.845) (end 143.25 88.295) (width 0.4) (layer "F.Cu") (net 4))
 (segment (start 153.1 121.245) (end 153.62 121.245) (width 0.4) (layer "F.Cu") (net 4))
 (segment (start 156.2 67.195) (end 156.2 67.547) (width 0.2) (layer "F.Cu") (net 4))
 (segment (start 145.225 118.745) (end 145.225 121.49) (width 0.4) (layer "F.Cu") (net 4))
 (segment (start 145.225 117.645) (end 145.225 118.745) (width 0.4) (layer "F.Cu") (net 4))
 (segment (start 143.25 88.295) (end 143.25 81.195) (width 0.4) (layer "F.Cu") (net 4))
 (segment (start 151.539 116.206) (end 152.9 114.845) (width 0.4) (layer "F.Cu") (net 4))
 (segment (start 144.65 115.195) (end 144.65 117.07) (width 0.4) (layer "F.Cu") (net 4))
 (segment (start 158.2 69.547) (end 157.802 69.945) (width 0.4) (layer "F.Cu") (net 4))
 (segment (start 153.62 121.245) (end 154.22 121.845) (width 0.4) (layer "F.Cu") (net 4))
 (segment (start 157.25 69.945) (end 157 69.945) (width 0.2) (layer "F.Cu") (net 4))
 (segment (start 144.65 117.07) (end 145.225 117.645) (width 0.4) (layer "F.Cu") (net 4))
 (segment (start 151.539 117.319) (end 151.539 116.206) (width 0.4) (layer "F.Cu") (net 4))
 (segment (start 154.9 113.345) (end 156.2 114.645) (width 0.2) (layer "F.Cu") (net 4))
 (segment (start 153.065 118.845) (end 151.539 117.319) (width 0.3) (layer "F.Cu") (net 4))
 (segment (start 145.225 121.49) (end 145.58 121.845) (width 0.2) (layer "F.Cu") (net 4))
 (segment (start 157.7 67.195) (end 158.2 67.695) (width 0.4) (layer "F.Cu") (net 4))
 (segment (start 151.900062 102.224938) (end 151.900062 114.345062) (width 0.4) (layer "F.Cu") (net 4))
 (segment (start 153.65 70.795) (end 151.9 72.545) (width 0.4) (layer "F.Cu") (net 4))
 (segment (start 157.25 70.795) (end 153.65 70.795) (width 0.4) (layer "F.Cu") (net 4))
 (segment (start 151.900062 114.345062) (end 152.4 114.845) (width 0.4) (layer "F.Cu") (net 4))
 (segment (start 154.9 99.225) (end 151.900062 102.224938) (width 0.4) (layer "F.Cu") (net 4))
 (segment (start 153.1 121.245) (end 153.1 118.88) (width 0.4) (layer "F.Cu") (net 4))
 (segment (start 152.875 118.845) (end 153.1 119.07) (width 0.2) (layer "F.Cu") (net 4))
 (segment (start 143.25 81.195) (end 143.25 81.145) (width 0.2) (layer "F.Cu") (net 4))
 (segment (start 144.1 112.995) (end 144.1 114.645) (width 0.4) (layer "F.Cu") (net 4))
 (segment (start 146.7 121.245) (end 146.18 121.245) (width 0.2) (layer "F.Cu") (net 4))
 (segment (start 154.9 112.345) (end 152.4 114.845) (width 0.2) (layer "F.Cu") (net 4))
 (segment (start 158.2 67.695) (end 158.2 69.547) (width 0.4) (layer "F.Cu") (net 4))
 (segment (start 145.8 90.845) (end 145.8 98.745) (width 0.4) (layer "F.Cu") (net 4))
 (segment (start 148.6 75.845) (end 143.25 81.195) (width 0.2) (layer "F.Cu") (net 4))
 (segment (start 157.25 69.945) (end 157.25 70.795) (width 0.4) (layer "F.Cu") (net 4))
 (segment (start 151.9 75.845) (end 157.25 81.195) (width 0.2) (layer "F.Cu") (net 4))
 (segment (start 154.22 126.045) (end 154.22 121.845) (width 0.4) (layer "F.Cu") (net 4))
 (segment (start 157.25 67.195) (end 157.7 67.195) (width 0.2) (layer "F.Cu") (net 4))
 (segment (start 154.9 99.225) (end 146.52 90.845) (width 0.2) (layer "B.Cu") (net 4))
 (segment (start 146.52 90.845) (end 145.8 90.845) (width 0.2) (layer "B.Cu") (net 4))
 (segment (start 151.65 119.24) (end 152.045 118.845) (width 0.2) (layer "F.Cu") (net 46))
 (segment (start 151.65 121.245) (end 151.65 119.24) (width 0.2) (layer "F.Cu") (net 46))
 (segment (start 153.65 81.195) (end 153.65 90.595) (width 0.4) (layer "F.Cu") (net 5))
 (segment (start 153.65 90.595) (end 153.4 90.845) (width 0.2) (layer "F.Cu") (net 5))
 (segment (start 150.65 122.117) (end 150.65 121.245) (width 0.2) (layer "F.Cu") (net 28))
 (segment (start 150.65 81.845) (end 150.65 121.245) (width 0.2) (layer "F.Cu") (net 28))
 (segment (start 151.1 81.195) (end 151.1 81.395) (width 0.2) (layer "F.Cu") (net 28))
 (segment (start 150.601 122.166) (end 150.65 122.117) (width 0.2) (layer "F.Cu") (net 28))
 (segment (start 149.699 122.166) (end 150.601 122.166) (width 0.2) (layer "F.Cu") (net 28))
 (segment (start 149.65 121.245) (end 149.65 122.117) (width 0.2) (layer "F.Cu") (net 28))
 (segment (start 149.65 122.117) (end 149.699 122.166) (width 0.2) (layer "F.Cu") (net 28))
 (segment (start 151.1 81.395) (end 150.65 81.845) (width 0.2) (layer "F.Cu") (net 28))
 (segment (start 146.4 119.845) (end 146.4 118.9) (width 0.2) (layer "F.Cu") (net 6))
 (segment (start 146.375 119.82) (end 146.4 119.845) (width 0.2) (layer "F.Cu") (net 6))
 (segment (start 148.65 120.095) (end 148.4 119.845) (width 0.2) (layer "F.Cu") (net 6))
 (segment (start 146.4 118.9) (end 146.245 118.745) (width 0.2) (layer "F.Cu") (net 6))
 (segment (start 148.65 121.245) (end 148.65 120.095) (width 0.2) (layer "F.Cu") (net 6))
 (via (at 148.4 119.845) (size 0.7) (drill 0.3) (layers "F.Cu" "B.Cu") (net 6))
 (via (at 146.4 119.845) (size 0.7) (drill 0.3) (layers "F.Cu" "B.Cu") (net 6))
 (segment (start 148.4 119.845) (end 146.4 119.845) (width 0.4) (layer "B.Cu") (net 6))
 (segment (start 150.15 119.373) (end 149.15 120.373) (width 0.2) (layer "F.Cu") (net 27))
 (segment (start 150.15 119.845) (end 150.15 121.245) (width 0.2) (layer "F.Cu") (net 27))
 (segment (start 150.15 81.295) (end 150.15 119.195) (width 0.2) (layer "F.Cu") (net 27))
 (segment (start 150.15 119.195) (end 150.15 119.373) (width 0.2) (layer "F.Cu") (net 27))
 (segment (start 150.25 81.195) (end 150.15 81.295) (width 0.2) (layer "F.Cu") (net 27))
 (segment (start 149.15 120.373) (end 149.15 121.245) (width 0.2) (layer "F.Cu") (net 27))
 (segment (start 150.15 119.195) (end 150.15 119.845) (width 0.2) (layer "F.Cu") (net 27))
 (segment (start 152.8 116.345) (end 152.4 116.745) (width 0.2) (layer "F.Cu") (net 1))
 (segment (start 155.85 116.845) (end 156.2 117.195) (width 0.2) (layer "F.Cu") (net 1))
 (segment (start 154.4 116.845) (end 155.85 116.845) (width 0.4) (layer "F.Cu") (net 1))
 (segment (start 148.7 115.6075) (end 148.7 112.995) (width 0.4) (layer "F.Cu") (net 1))
 (segment (start 149.4 116.345) (end 147.9625 116.345) (width 0.4) (layer "F.Cu") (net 1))
 (segment (start 147.9625 116.345) (end 147.9 116.4075) (width 0.2) (layer "F.Cu") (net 1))
 (segment (start 157.2 115.895) (end 157.2 111.195) (width 0.4) (layer "F.Cu") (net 1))
 (segment (start 157.2 115.935) (end 157.2 115.895) (width 0.2) (layer "F.Cu") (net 1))
 (segment (start 154.4 116.845) (end 153 116.845) (width 0.4) (layer "F.Cu") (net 1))
 (segment (start 147.9 116.4075) (end 148.7 115.6075) (width 0.4) (layer "F.Cu") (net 1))
 (segment (start 156.19 116.945) (end 157.2 115.935) (width 0.4) (layer "F.Cu") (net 1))
 (segment (start 153 116.845) (end 152.9 116.745) (width 0.2) (layer "F.Cu") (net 1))
 (via (at 149.4 116.345) (size 0.7) (drill 0.3) (layers "F.Cu" "B.Cu") (free yes) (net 1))
 (via (at 154.4 116.845) (size 0.7) (drill 0.3) (layers "F.Cu" "B.Cu") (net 1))
 (segment (start 149.4 116.345) (end 149.9 116.845) (width 0.4) (layer "B.Cu") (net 1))
 (segment (start 149.9 116.845) (end 154.4 116.845) (width 0.4) (layer "B.Cu") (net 1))
 (segment (start 145.875 113.52) (end 146.4 112.995) (width 0.2) (layer "F.Cu") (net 7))
 (segment (start 146.4 106.695) (end 147.4 105.695) (width 0.2) (layer "F.Cu") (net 7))
 (segment (start 142.301 102.596) (end 142.301 70.195) (width 0.4) (layer "F.Cu") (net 7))
 (segment (start 143.25 69.945) (end 153.8 69.945) (width 0.381) (layer "F.Cu") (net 7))
 (segment (start 146.4 106.695) (end 142.301 102.596) (width 0.4) (layer "F.Cu") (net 7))
 (segment (start 146.4 106.695) (end 146.4 112.995) (width 0.8) (layer "F.Cu") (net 7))
 (segment (start 155.5 68.245) (end 157.25 68.245) (width 0.381) (layer "F.Cu") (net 7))
 (segment (start 153.8 69.945) (end 155.5 68.245) (width 0.381) (layer "F.Cu") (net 7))
 (segment (start 142.551 69.945) (end 143.25 69.945) (width 0.4) (layer "F.Cu") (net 7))
 (segment (start 146.2 113.195) (end 146.4 112.995) (width 0.2) (layer "F.Cu") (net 7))
 (segment (start 147.4 105.695) (end 147.4 102.345) (width 0.2) (layer "F.Cu") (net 7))
 (segment (start 142.301 70.195) (end 142.551 69.945) (width 0.4) (layer "F.Cu") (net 7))
 (segment (start 146.2 115.195) (end 146.2 113.195) (width 0.2) (layer "F.Cu") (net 7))
 (segment (start 144.86 102.345) (end 144.86 98.865) (width 0.2) (layer "F.Cu") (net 47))
 (segment (start 144.86 98.865) (end 144.88 98.845) (width 0.2) (layer "F.Cu") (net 47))
 (segment (start 147.686 122.153) (end 148.1 122.567) (width 0.2) (layer "F.Cu") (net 45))
 (segment (start 147.686 121.431) (end 147.686 122.153) (width 0.2) (layer "F.Cu") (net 45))
 (segment (start 147.5 121.245) (end 147.5 119.1825) (width 0.2) (layer "F.Cu") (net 45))
 (segment (start 147.5 121.245) (end 147.686 121.431) (width 0.2) (layer "F.Cu") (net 45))
 (segment (start 148.1 122.567) (end 151.631992 122.567) (width 0.2) (layer "F.Cu") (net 45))
 (segment (start 147.9 118.2825) (end 147.9 118.7825) (width 0.2) (layer "F.Cu") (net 45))
 (segment (start 151.631992 122.567) (end 152.3 121.898992) (width 0.2) (layer "F.Cu") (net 45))
 (segment (start 152.3 121.898992) (end 152.3 121.245) (width 0.2) (layer "F.Cu") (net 45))
 (segment (start 147.9 118.7825) (end 147.5 119.1825) (width 0.2) (layer "F.Cu") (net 45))
 (segment (start 156.2 103.005) (end 154.9 104.305) (width 0.4) (layer "F.Cu") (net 2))
 (segment (start 156.2 81.195) (end 156.2 103.005) (width 0.4) (layer "F.Cu") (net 2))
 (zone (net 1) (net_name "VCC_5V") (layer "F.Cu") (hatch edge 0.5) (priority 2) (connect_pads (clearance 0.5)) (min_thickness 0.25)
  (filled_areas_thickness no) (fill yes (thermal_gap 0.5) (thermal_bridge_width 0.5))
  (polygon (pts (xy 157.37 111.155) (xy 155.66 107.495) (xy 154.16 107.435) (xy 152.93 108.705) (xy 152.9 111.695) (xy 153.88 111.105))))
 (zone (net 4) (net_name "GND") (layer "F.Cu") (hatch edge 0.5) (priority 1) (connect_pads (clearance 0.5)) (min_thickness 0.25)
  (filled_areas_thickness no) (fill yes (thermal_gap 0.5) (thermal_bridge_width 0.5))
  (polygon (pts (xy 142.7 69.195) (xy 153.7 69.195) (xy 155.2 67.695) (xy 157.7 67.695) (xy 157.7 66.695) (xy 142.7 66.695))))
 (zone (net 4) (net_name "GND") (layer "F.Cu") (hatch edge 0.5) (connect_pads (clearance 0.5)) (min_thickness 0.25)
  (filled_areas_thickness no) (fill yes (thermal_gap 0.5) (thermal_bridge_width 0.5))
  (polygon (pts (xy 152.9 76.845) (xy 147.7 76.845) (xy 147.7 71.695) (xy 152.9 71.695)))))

